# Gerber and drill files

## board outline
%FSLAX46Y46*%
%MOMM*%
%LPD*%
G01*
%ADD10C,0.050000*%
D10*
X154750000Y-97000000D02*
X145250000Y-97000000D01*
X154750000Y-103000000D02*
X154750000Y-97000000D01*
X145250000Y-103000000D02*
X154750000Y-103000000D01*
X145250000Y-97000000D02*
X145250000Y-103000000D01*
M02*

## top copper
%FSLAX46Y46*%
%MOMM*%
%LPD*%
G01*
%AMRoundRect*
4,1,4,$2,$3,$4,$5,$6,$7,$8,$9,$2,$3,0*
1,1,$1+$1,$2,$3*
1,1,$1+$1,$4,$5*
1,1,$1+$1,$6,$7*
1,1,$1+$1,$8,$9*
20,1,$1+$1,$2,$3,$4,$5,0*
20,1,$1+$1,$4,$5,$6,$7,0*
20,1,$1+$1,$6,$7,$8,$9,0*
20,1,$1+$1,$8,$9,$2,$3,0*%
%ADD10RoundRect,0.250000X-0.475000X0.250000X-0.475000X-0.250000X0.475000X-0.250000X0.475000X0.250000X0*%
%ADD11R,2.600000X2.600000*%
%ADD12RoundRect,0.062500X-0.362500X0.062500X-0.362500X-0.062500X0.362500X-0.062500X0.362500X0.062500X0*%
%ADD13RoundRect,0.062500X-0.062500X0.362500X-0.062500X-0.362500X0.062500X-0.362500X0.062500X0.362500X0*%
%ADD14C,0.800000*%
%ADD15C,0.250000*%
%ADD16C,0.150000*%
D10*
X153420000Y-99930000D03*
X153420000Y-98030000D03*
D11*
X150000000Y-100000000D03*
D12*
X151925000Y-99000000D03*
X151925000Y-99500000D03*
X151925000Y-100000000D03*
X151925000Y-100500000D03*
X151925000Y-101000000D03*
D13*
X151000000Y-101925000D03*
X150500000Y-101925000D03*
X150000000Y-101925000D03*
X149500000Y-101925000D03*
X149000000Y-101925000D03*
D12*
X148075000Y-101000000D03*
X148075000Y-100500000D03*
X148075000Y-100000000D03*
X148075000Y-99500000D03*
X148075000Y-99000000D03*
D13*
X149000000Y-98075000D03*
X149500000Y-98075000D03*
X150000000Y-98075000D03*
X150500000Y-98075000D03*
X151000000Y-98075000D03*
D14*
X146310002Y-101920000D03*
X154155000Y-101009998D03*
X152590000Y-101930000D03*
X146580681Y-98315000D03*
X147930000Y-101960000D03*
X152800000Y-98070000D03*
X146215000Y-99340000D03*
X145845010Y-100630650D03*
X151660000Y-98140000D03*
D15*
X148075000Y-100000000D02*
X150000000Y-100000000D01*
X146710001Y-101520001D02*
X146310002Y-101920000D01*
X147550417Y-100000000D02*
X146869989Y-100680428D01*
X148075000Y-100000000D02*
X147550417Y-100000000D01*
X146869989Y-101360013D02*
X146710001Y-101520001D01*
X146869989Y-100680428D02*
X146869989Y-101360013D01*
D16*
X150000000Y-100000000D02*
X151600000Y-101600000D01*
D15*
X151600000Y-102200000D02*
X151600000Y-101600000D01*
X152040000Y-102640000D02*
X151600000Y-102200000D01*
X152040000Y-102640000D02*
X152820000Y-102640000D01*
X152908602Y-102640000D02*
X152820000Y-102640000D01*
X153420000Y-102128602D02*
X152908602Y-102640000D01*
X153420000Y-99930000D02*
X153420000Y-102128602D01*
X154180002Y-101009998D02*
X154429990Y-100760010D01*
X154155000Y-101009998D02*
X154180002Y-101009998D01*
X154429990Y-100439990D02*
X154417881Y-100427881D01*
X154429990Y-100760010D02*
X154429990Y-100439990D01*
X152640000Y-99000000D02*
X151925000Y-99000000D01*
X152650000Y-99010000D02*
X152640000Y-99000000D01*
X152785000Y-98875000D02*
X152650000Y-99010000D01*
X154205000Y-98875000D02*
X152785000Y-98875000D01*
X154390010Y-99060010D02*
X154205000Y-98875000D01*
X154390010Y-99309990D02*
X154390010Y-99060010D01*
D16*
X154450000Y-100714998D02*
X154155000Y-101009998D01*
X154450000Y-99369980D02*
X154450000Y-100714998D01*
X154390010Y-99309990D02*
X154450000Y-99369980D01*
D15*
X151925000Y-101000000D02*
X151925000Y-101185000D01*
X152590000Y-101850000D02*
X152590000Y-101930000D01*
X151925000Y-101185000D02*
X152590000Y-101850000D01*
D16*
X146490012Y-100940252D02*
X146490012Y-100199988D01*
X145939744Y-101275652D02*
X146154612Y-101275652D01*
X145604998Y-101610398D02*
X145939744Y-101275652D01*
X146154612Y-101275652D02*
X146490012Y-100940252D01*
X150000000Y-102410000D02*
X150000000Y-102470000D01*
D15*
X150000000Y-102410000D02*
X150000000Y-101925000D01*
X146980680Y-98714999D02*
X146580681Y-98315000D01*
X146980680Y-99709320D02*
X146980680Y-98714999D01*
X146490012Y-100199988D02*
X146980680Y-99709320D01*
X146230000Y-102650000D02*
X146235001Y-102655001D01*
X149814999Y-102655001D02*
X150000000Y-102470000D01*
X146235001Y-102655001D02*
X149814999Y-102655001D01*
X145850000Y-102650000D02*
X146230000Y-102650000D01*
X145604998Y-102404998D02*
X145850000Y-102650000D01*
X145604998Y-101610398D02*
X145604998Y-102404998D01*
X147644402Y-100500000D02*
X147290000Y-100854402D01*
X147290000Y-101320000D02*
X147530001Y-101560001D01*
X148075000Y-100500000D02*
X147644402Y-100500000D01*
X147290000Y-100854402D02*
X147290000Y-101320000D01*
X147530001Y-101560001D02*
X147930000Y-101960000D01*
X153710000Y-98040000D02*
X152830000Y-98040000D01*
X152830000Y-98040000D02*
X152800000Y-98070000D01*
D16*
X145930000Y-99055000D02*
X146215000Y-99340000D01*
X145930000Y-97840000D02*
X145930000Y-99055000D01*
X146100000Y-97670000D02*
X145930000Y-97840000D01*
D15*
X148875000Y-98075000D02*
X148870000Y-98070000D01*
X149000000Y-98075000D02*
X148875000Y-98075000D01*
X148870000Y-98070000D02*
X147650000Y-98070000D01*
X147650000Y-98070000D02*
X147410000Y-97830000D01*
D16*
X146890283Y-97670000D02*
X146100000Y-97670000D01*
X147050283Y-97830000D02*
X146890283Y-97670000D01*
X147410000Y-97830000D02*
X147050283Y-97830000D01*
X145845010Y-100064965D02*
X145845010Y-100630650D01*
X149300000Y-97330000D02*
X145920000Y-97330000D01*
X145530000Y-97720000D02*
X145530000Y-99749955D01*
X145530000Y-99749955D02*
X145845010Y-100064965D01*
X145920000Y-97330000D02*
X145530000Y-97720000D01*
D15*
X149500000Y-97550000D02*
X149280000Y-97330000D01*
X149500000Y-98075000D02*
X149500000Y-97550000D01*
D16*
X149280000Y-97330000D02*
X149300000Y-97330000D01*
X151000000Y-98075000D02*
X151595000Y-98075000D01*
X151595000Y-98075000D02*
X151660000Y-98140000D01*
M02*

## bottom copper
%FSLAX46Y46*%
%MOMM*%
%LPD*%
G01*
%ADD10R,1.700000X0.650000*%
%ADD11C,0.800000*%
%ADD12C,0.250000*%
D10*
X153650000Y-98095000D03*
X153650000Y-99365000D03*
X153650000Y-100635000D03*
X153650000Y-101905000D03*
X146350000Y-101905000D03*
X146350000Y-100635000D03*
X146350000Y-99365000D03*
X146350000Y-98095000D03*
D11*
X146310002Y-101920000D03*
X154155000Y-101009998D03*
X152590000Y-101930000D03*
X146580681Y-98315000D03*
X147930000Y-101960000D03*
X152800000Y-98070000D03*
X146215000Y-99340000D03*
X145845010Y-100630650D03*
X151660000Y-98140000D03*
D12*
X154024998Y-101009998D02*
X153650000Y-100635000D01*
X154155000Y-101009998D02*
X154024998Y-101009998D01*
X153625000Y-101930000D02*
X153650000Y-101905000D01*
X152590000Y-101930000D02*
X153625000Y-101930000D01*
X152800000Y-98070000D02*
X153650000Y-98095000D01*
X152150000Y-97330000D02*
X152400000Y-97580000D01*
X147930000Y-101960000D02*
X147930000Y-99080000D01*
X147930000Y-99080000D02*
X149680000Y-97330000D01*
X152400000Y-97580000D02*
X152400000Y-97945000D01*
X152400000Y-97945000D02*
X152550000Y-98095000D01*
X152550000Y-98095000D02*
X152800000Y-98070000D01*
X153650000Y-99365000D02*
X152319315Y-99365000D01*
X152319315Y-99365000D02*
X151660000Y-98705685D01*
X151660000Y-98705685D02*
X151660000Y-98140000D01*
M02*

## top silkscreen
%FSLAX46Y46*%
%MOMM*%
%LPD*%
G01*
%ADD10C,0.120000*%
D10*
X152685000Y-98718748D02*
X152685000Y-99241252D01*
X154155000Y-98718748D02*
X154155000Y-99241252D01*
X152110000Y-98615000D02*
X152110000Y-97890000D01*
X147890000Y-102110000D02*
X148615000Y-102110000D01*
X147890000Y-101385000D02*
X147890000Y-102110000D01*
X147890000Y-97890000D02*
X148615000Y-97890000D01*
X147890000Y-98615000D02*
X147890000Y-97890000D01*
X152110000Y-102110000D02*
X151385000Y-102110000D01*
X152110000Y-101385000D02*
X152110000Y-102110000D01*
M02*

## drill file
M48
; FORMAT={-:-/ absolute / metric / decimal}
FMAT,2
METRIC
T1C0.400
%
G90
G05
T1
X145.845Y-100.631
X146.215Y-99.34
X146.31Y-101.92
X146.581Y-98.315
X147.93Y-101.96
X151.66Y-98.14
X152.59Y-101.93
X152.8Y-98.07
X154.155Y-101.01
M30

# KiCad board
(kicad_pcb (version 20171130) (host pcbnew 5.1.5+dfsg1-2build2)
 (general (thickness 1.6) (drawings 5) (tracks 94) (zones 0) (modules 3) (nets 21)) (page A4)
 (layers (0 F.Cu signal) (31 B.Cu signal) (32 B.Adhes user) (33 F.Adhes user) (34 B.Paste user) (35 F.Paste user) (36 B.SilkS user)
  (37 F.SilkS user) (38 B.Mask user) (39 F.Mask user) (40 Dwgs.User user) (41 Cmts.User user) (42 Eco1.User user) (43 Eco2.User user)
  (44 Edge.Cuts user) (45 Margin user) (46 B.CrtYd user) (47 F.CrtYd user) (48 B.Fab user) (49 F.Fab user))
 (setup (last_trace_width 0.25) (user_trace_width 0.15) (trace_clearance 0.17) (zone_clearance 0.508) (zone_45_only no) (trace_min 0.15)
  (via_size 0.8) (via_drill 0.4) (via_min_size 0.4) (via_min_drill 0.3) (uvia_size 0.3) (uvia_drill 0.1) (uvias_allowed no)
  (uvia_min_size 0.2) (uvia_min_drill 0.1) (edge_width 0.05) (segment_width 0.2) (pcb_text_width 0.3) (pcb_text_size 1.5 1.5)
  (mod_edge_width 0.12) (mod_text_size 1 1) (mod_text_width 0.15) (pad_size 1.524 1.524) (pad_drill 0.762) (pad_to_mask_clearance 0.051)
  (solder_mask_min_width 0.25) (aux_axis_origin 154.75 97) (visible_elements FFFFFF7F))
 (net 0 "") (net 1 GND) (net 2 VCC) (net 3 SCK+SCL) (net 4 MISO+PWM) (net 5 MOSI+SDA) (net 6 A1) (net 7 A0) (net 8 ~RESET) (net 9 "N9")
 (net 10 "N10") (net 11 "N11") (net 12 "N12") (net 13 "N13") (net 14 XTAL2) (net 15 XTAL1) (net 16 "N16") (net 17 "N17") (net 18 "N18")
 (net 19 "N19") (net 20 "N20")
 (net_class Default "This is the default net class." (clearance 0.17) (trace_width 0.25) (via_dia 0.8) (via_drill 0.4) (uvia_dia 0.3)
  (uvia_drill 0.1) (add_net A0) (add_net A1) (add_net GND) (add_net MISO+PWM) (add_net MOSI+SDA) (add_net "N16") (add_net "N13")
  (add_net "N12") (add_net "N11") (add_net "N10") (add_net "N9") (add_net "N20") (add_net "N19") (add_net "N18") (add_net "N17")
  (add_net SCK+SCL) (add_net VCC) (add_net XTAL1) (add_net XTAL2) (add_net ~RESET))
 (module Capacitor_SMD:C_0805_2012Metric (layer F.Cu) (at 153.42 98.98 270)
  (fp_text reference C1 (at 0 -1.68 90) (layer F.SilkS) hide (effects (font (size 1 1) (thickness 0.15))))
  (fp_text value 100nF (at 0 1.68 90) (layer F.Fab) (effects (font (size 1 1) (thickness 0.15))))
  (fp_line (start -0.261252 0.735) (end 0.261252 0.735) (layer F.SilkS) (width 0.12))
  (fp_line (start -0.261252 -0.735) (end 0.261252 -0.735) (layer F.SilkS) (width 0.12))
  (pad 2 smd roundrect (at 0.95 0 270) (size 1 1.45) (layers F.Cu F.Paste F.Mask) (roundrect_rratio 0.25) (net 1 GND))
  (pad 1 smd roundrect (at -0.95 0 270) (size 1 1.45) (layers F.Cu F.Paste F.Mask) (roundrect_rratio 0.25) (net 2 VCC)))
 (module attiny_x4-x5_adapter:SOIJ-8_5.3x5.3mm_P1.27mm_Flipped (layer F.Cu) (at 150 100)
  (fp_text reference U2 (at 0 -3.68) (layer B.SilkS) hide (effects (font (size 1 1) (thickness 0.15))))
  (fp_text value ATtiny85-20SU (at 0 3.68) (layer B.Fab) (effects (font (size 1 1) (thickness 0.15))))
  (pad 8 smd rect (at 3.65 -1.905) (size 1.7 0.65) (layers B.Cu B.Paste B.Mask) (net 2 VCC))
  (pad 7 smd rect (at 3.65 -0.635) (size 1.7 0.65) (layers B.Cu B.Paste B.Mask) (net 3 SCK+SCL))
  (pad 6 smd rect (at 3.65 0.635) (size 1.7 0.65) (layers B.Cu B.Paste B.Mask) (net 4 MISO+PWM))
  (pad 5 smd rect (at 3.65 1.905) (size 1.7 0.65) (layers B.Cu B.Paste B.Mask) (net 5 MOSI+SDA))
  (pad 4 smd rect (at -3.65 1.905) (size 1.7 0.65) (layers B.Cu B.Paste B.Mask) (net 1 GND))
  (pad 3 smd rect (at -3.65 0.635) (size 1.7 0.65) (layers B.Cu B.Paste B.Mask) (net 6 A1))
  (pad 2 smd rect (at -3.65 -0.635) (size 1.7 0.65) (layers B.Cu B.Paste B.Mask) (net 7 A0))
  (pad 1 smd rect (at -3.65 -1.905) (size 1.7 0.65) (layers B.Cu B.Paste B.Mask) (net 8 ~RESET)))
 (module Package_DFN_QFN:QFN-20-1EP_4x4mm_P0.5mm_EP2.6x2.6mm (layer F.Cu) (at 150 100 270)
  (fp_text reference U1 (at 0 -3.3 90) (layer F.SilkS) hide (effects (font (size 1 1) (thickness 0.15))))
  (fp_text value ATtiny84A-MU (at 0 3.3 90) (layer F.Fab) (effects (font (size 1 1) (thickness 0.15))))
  (fp_line (start -1.385 -2.11) (end -2.11 -2.11) (layer F.SilkS) (width 0.12))
  (fp_line (start 2.11 2.11) (end 2.11 1.385) (layer F.SilkS) (width 0.12))
  (fp_line (start 1.385 2.11) (end 2.11 2.11) (layer F.SilkS) (width 0.12))
  (fp_line (start -2.11 2.11) (end -2.11 1.385) (layer F.SilkS) (width 0.12))
  (fp_line (start -1.385 2.11) (end -2.11 2.11) (layer F.SilkS) (width 0.12))
  (fp_line (start 2.11 -2.11) (end 2.11 -1.385) (layer F.SilkS) (width 0.12))
  (fp_line (start 1.385 -2.11) (end 2.11 -2.11) (layer F.SilkS) (width 0.12))
  (pad "" smd roundrect (at 0.65 0.65 270) (size 1.05 1.05) (layers F.Paste) (roundrect_rratio 0.238095))
  (pad "" smd roundrect (at 0.65 -0.65 270) (size 1.05 1.05) (layers F.Paste) (roundrect_rratio 0.238095))
  (pad "" smd roundrect (at -0.65 0.65 270) (size 1.05 1.05) (layers F.Paste) (roundrect_rratio 0.238095))
  (pad "" smd roundrect (at -0.65 -0.65 270) (size 1.05 1.05) (layers F.Paste) (roundrect_rratio 0.238095))
  (pad 21 smd rect (at 0 0 270) (size 2.6 2.6) (layers F.Cu F.Mask) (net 1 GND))
  (pad 20 smd roundrect (at -1 -1.925 270) (size 0.25 0.85) (layers F.Cu F.Paste F.Mask) (roundrect_rratio 0.25) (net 4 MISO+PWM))
  (pad 19 smd roundrect (at -0.5 -1.925 270) (size 0.25 0.85) (layers F.Cu F.Paste F.Mask) (roundrect_rratio 0.25) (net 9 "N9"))
  (pad 18 smd roundrect (at 0 -1.925 270) (size 0.25 0.85) (layers F.Cu F.Paste F.Mask) (roundrect_rratio 0.25) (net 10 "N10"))
  (pad 17 smd roundrect (at 0.5 -1.925 270) (size 0.25 0.85) (layers F.Cu F.Paste F.Mask) (roundrect_rratio 0.25) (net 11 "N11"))
  (pad 16 smd roundrect (at 1 -1.925 270) (size 0.25 0.85) (layers F.Cu F.Paste F.Mask) (roundrect_rratio 0.25) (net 5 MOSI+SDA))
  (pad 15 smd roundrect (at 1.925 -1 270) (size 0.85 0.25) (layers F.Cu F.Paste F.Mask) (roundrect_rratio 0.25) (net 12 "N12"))
  (pad 14 smd roundrect (at 1.925 -0.5 270) (size 0.85 0.25) (layers F.Cu F.Paste F.Mask) (roundrect_rratio 0.25) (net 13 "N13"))
  (pad 13 smd roundrect (at 1.925 0 270) (size 0.85 0.25) (layers F.Cu F.Paste F.Mask) (roundrect_rratio 0.25) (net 8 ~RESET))
  (pad 12 smd roundrect (at 1.925 0.5 270) (size 0.85 0.25) (layers F.Cu F.Paste F.Mask) (roundrect_rratio 0.25) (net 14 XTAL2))
  (pad 11 smd roundrect (at 1.925 1 270) (size 0.85 0.25) (layers F.Cu F.Paste F.Mask) (roundrect_rratio 0.25) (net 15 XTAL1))
  (pad 10 smd roundrect (at 1 1.925 270) (size 0.25 0.85) (layers F.Cu F.Paste F.Mask) (roundrect_rratio 0.25) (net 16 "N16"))
  (pad 9 smd roundrect (at 0.5 1.925 270) (size 0.25 0.85) (layers F.Cu F.Paste F.Mask) (roundrect_rratio 0.25) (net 2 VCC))
  (pad 8 smd roundrect (at 0 1.925 270) (size 0.25 0.85) (layers F.Cu F.Paste F.Mask) (roundrect_rratio 0.25) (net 1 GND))
  (pad 7 smd roundrect (at -0.5 1.925 270) (size 0.25 0.85) (layers F.Cu F.Paste F.Mask) (roundrect_rratio 0.25) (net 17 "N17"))
  (pad 6 smd roundrect (at -1 1.925 270) (size 0.25 0.85) (layers F.Cu F.Paste F.Mask) (roundrect_rratio 0.25) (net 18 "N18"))
  (pad 5 smd roundrect (at -1.925 1 270) (size 0.85 0.25) (layers F.Cu F.Paste F.Mask) (roundrect_rratio 0.25) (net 7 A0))
  (pad 4 smd roundrect (at -1.925 0.5 270) (size 0.85 0.25) (layers F.Cu F.Paste F.Mask) (roundrect_rratio 0.25) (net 6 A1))
  (pad 3 smd roundrect (at -1.925 0 270) (size 0.85 0.25) (layers F.Cu F.Paste F.Mask) (roundrect_rratio 0.25) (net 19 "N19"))
  (pad 2 smd roundrect (at -1.925 -0.5 270) (size 0.85 0.25) (layers F.Cu F.Paste F.Mask) (roundrect_rratio 0.25) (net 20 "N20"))
  (pad 1 smd roundrect (at -1.925 -1 270) (size 0.85 0.25) (layers F.Cu F.Paste F.Mask) (roundrect_rratio 0.25) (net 3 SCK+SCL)))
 (gr_line (start 154.75 97) (end 145.25 97) (layer Edge.Cuts) (width 0.05))
 (gr_line (start 154.75 103) (end 154.75 97) (layer Edge.Cuts) (width 0.05))
 (gr_line (start 145.25 103) (end 154.75 103) (layer Edge.Cuts) (width 0.05))
 (gr_line (start 145.25 97) (end 145.25 103) (layer Edge.Cuts) (width 0.05))
 (segment (start 148.075 100) (end 150 100) (width 0.25) (layer F.Cu) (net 1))
 (segment (start 146.710001 101.520001) (end 146.310002 101.92) (width 0.25) (layer F.Cu) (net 1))
 (segment (start 147.550417 100) (end 146.869989 100.680428) (width 0.25) (layer F.Cu) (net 1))
 (segment (start 148.075 100) (end 147.550417 100) (width 0.25) (layer F.Cu) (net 1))
 (via (at 146.310002 101.92) (size 0.8) (drill 0.4) (layers F.Cu B.Cu) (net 1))
 (segment (start 146.869989 101.360013) (end 146.710001 101.520001) (width 0.25) (layer F.Cu) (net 1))
 (segment (start 146.869989 100.680428) (end 146.869989 101.360013) (width 0.25) (layer F.Cu) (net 1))
 (segment (start 150 100) (end 151.6 101.6) (width 0.15) (layer F.Cu) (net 1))
 (segment (start 151.6 102.2) (end 151.6 101.6) (width 0.25) (layer F.Cu) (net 1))
 (segment (start 152.04 102.64) (end 151.6 102.2) (width 0.25) (layer F.Cu) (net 1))
 (segment (start 152.04 102.64) (end 152.82 102.64) (width 0.25) (layer F.Cu) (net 1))
 (segment (start 152.908602 102.64) (end 152.82 102.64) (width 0.25) (layer F.Cu) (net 1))
 (segment (start 153.42 102.128602) (end 152.908602 102.64) (width 0.25) (layer F.Cu) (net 1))
 (segment (start 153.42 99.93) (end 153.42 102.128602) (width 0.25) (layer F.Cu) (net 1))
 (via (at 154.155 101.009998) (size 0.8) (drill 0.4) (layers F.Cu B.Cu) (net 4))
 (segment (start 154.024998 101.009998) (end 153.65 100.635) (width 0.25) (layer B.Cu) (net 4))
 (segment (start 154.155 101.009998) (end 154.024998 101.009998) (width 0.25) (layer B.Cu) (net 4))
 (segment (start 154.180002 101.009998) (end 154.42999 100.76001) (width 0.25) (layer F.Cu) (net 4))
 (segment (start 154.155 101.009998) (end 154.180002 101.009998) (width 0.25) (layer F.Cu) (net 4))
 (segment (start 154.42999 100.43999) (end 154.417881 100.427881) (width 0.25) (layer F.Cu) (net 4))
 (segment (start 154.42999 100.76001) (end 154.42999 100.43999) (width 0.25) (layer F.Cu) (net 4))
 (segment (start 152.64 99) (end 151.925 99) (width 0.25) (layer F.Cu) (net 4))
 (segment (start 152.65 99.01) (end 152.64 99) (width 0.25) (layer F.Cu) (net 4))
 (segment (start 152.785 98.875) (end 152.65 99.01) (width 0.25) (layer F.Cu) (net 4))
 (segment (start 154.205 98.875) (end 152.785 98.875) (width 0.25) (layer F.Cu) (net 4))
 (segment (start 154.39001 99.06001) (end 154.205 98.875) (width 0.25) (layer F.Cu) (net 4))
 (segment (start 154.39001 99.30999) (end 154.39001 99.06001) (width 0.25) (layer F.Cu) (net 4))
 (segment (start 154.45 100.714998) (end 154.155 101.009998) (width 0.15) (layer F.Cu) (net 4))
 (segment (start 154.45 99.36998) (end 154.45 100.714998) (width 0.15) (layer F.Cu) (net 4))
 (segment (start 154.39001 99.30999) (end 154.45 99.36998) (width 0.15) (layer F.Cu) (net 4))
 (segment (start 151.925 101) (end 151.925 101.185) (width 0.25) (layer F.Cu) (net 5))
 (via (at 152.59 101.93) (size 0.8) (drill 0.4) (layers F.Cu B.Cu) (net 5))
 (segment (start 152.59 101.85) (end 152.59 101.93) (width 0.25) (layer F.Cu) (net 5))
 (segment (start 151.925 101.185) (end 152.59 101.85) (width 0.25) (layer F.Cu) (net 5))
 (segment (start 153.625 101.93) (end 153.65 101.905) (width 0.25) (layer B.Cu) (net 5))
 (segment (start 152.59 101.93) (end 153.625 101.93) (width 0.25) (layer B.Cu) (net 5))
 (via (at 146.580681 98.315) (size 0.8) (drill 0.4) (layers F.Cu B.Cu) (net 8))
 (segment (start 146.490012 100.940252) (end 146.490012 100.199988) (width 0.15) (layer F.Cu) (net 8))
 (segment (start 145.939744 101.275652) (end 146.154612 101.275652) (width 0.15) (layer F.Cu) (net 8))
 (segment (start 145.604998 101.610398) (end 145.939744 101.275652) (width 0.15) (layer F.Cu) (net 8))
 (segment (start 146.154612 101.275652) (end 146.490012 100.940252) (width 0.15) (layer F.Cu) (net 8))
 (segment (start 150 102.41) (end 150 102.47) (width 0.15) (layer F.Cu) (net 8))
 (segment (start 150 102.41) (end 150 101.925) (width 0.25) (layer F.Cu) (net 8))
 (segment (start 146.98068 98.714999) (end 146.580681 98.315) (width 0.25) (layer F.Cu) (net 8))
 (segment (start 146.98068 99.70932) (end 146.98068 98.714999) (width 0.25) (layer F.Cu) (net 8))
 (segment (start 146.490012 100.199988) (end 146.98068 99.70932) (width 0.25) (layer F.Cu) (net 8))
 (segment (start 146.23 102.65) (end 146.235001 102.655001) (width 0.25) (layer F.Cu) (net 8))
 (segment (start 149.814999 102.655001) (end 150 102.47) (width 0.25) (layer F.Cu) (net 8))
 (segment (start 146.235001 102.655001) (end 149.814999 102.655001) (width 0.25) (layer F.Cu) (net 8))
 (segment (start 145.85 102.65) (end 146.23 102.65) (width 0.25) (layer F.Cu) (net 8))
 (segment (start 145.604998 102.404998) (end 145.85 102.65) (width 0.25) (layer F.Cu) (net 8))
 (segment (start 145.604998 101.610398) (end 145.604998 102.404998) (width 0.25) (layer F.Cu) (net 8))
 (via (at 147.93 101.96) (size 0.8) (drill 0.4) (layers F.Cu B.Cu) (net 2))
 (segment (start 147.644402 100.5) (end 147.29 100.854402) (width 0.25) (layer F.Cu) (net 2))
 (segment (start 147.29 101.32) (end 147.530001 101.560001) (width 0.25) (layer F.Cu) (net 2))
 (segment (start 148.075 100.5) (end 147.644402 100.5) (width 0.25) (layer F.Cu) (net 2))
 (segment (start 147.29 100.854402) (end 147.29 101.32) (width 0.25) (layer F.Cu) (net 2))
 (segment (start 147.530001 101.560001) (end 147.93 101.96) (width 0.25) (layer F.Cu) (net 2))
 (via (at 152.8 98.07) (size 0.8) (drill 0.4) (layers F.Cu B.Cu) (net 2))
 (segment (start 153.71 98.04) (end 152.83 98.04) (width 0.25) (layer F.Cu) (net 2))
 (segment (start 152.83 98.04) (end 152.8 98.07) (width 0.25) (layer F.Cu) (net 2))
 (segment (start 152.8 98.07) (end 153.65 98.095) (width 0.25) (layer B.Cu) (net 2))
 (segment (start 152.15 97.33) (end 152.4 97.58) (width 0.25) (layer B.Cu) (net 2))
 (segment (start 147.93 101.96) (end 147.93 99.08) (width 0.25) (layer B.Cu) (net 2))
 (segment (start 147.93 99.08) (end 149.68 97.33) (width 0.25) (layer B.Cu) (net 2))
 (segment (start 152.4 97.58) (end 152.4 97.945) (width 0.25) (layer B.Cu) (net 2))
 (segment (start 152.4 97.945) (end 152.55 98.095) (width 0.25) (layer B.Cu) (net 2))
 (segment (start 152.55 98.095) (end 152.8 98.07) (width 0.25) (layer B.Cu) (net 2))
 (via (at 146.215 99.34) (size 0.8) (drill 0.4) (layers F.Cu B.Cu) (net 7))
 (segment (start 145.93 99.055) (end 146.215 99.34) (width 0.15) (layer F.Cu) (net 7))
 (segment (start 145.93 97.84) (end 145.93 99.055) (width 0.15) (layer F.Cu) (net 7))
 (segment (start 146.1 97.67) (end 145.93 97.84) (width 0.15) (layer F.Cu) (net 7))
 (segment (start 148.875 98.075) (end 148.87 98.07) (width 0.25) (layer F.Cu) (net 7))
 (segment (start 149 98.075) (end 148.875 98.075) (width 0.25) (layer F.Cu) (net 7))
 (segment (start 148.87 98.07) (end 147.65 98.07) (width 0.25) (layer F.Cu) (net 7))
 (segment (start 147.65 98.07) (end 147.41 97.83) (width 0.25) (layer F.Cu) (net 7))
 (segment (start 146.890283 97.67) (end 146.1 97.67) (width 0.15) (layer F.Cu) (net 7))
 (segment (start 147.050283 97.83) (end 146.890283 97.67) (width 0.15) (layer F.Cu) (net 7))
 (segment (start 147.41 97.83) (end 147.050283 97.83) (width 0.15) (layer F.Cu) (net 7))
 (via (at 145.84501 100.63065) (size 0.8) (drill 0.4) (layers F.Cu B.Cu) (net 6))
 (segment (start 145.84501 100.064965) (end 145.84501 100.63065) (width 0.15) (layer F.Cu) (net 6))
 (segment (start 149.3 97.33) (end 145.92 97.33) (width 0.15) (layer F.Cu) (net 6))
 (segment (start 145.53 97.72) (end 145.53 99.749955) (width 0.15) (layer F.Cu) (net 6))
 (segment (start 145.53 99.749955) (end 145.84501 100.064965) (width 0.15) (layer F.Cu) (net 6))
 (segment (start 145.92 97.33) (end 145.53 97.72) (width 0.15) (layer F.Cu) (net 6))
 (segment (start 149.5 97.55) (end 149.28 97.33) (width 0.25) (layer F.Cu) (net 6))
 (segment (start 149.5 98.075) (end 149.5 97.55) (width 0.25) (layer F.Cu) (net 6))
 (segment (start 149.28 97.33) (end 149.3 97.33) (width 0.15) (layer F.Cu) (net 6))
 (via (at 151.66 98.14) (size 0.8) (drill 0.4) (layers F.Cu B.Cu) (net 3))
 (segment (start 151 98.075) (end 151.595 98.075) (width 0.15) (layer F.Cu) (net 3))
 (segment (start 151.595 98.075) (end 151.66 98.14) (width 0.15) (layer F.Cu) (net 3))
 (segment (start 153.65 99.365) (end 152.319315 99.365) (width 0.25) (layer B.Cu) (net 3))
 (segment (start 152.319315 99.365) (end 151.66 98.705685) (width 0.25) (layer B.Cu) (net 3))
 (segment (start 151.66 98.705685) (end 151.66 98.14) (width 0.25) (layer B.Cu) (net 3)))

